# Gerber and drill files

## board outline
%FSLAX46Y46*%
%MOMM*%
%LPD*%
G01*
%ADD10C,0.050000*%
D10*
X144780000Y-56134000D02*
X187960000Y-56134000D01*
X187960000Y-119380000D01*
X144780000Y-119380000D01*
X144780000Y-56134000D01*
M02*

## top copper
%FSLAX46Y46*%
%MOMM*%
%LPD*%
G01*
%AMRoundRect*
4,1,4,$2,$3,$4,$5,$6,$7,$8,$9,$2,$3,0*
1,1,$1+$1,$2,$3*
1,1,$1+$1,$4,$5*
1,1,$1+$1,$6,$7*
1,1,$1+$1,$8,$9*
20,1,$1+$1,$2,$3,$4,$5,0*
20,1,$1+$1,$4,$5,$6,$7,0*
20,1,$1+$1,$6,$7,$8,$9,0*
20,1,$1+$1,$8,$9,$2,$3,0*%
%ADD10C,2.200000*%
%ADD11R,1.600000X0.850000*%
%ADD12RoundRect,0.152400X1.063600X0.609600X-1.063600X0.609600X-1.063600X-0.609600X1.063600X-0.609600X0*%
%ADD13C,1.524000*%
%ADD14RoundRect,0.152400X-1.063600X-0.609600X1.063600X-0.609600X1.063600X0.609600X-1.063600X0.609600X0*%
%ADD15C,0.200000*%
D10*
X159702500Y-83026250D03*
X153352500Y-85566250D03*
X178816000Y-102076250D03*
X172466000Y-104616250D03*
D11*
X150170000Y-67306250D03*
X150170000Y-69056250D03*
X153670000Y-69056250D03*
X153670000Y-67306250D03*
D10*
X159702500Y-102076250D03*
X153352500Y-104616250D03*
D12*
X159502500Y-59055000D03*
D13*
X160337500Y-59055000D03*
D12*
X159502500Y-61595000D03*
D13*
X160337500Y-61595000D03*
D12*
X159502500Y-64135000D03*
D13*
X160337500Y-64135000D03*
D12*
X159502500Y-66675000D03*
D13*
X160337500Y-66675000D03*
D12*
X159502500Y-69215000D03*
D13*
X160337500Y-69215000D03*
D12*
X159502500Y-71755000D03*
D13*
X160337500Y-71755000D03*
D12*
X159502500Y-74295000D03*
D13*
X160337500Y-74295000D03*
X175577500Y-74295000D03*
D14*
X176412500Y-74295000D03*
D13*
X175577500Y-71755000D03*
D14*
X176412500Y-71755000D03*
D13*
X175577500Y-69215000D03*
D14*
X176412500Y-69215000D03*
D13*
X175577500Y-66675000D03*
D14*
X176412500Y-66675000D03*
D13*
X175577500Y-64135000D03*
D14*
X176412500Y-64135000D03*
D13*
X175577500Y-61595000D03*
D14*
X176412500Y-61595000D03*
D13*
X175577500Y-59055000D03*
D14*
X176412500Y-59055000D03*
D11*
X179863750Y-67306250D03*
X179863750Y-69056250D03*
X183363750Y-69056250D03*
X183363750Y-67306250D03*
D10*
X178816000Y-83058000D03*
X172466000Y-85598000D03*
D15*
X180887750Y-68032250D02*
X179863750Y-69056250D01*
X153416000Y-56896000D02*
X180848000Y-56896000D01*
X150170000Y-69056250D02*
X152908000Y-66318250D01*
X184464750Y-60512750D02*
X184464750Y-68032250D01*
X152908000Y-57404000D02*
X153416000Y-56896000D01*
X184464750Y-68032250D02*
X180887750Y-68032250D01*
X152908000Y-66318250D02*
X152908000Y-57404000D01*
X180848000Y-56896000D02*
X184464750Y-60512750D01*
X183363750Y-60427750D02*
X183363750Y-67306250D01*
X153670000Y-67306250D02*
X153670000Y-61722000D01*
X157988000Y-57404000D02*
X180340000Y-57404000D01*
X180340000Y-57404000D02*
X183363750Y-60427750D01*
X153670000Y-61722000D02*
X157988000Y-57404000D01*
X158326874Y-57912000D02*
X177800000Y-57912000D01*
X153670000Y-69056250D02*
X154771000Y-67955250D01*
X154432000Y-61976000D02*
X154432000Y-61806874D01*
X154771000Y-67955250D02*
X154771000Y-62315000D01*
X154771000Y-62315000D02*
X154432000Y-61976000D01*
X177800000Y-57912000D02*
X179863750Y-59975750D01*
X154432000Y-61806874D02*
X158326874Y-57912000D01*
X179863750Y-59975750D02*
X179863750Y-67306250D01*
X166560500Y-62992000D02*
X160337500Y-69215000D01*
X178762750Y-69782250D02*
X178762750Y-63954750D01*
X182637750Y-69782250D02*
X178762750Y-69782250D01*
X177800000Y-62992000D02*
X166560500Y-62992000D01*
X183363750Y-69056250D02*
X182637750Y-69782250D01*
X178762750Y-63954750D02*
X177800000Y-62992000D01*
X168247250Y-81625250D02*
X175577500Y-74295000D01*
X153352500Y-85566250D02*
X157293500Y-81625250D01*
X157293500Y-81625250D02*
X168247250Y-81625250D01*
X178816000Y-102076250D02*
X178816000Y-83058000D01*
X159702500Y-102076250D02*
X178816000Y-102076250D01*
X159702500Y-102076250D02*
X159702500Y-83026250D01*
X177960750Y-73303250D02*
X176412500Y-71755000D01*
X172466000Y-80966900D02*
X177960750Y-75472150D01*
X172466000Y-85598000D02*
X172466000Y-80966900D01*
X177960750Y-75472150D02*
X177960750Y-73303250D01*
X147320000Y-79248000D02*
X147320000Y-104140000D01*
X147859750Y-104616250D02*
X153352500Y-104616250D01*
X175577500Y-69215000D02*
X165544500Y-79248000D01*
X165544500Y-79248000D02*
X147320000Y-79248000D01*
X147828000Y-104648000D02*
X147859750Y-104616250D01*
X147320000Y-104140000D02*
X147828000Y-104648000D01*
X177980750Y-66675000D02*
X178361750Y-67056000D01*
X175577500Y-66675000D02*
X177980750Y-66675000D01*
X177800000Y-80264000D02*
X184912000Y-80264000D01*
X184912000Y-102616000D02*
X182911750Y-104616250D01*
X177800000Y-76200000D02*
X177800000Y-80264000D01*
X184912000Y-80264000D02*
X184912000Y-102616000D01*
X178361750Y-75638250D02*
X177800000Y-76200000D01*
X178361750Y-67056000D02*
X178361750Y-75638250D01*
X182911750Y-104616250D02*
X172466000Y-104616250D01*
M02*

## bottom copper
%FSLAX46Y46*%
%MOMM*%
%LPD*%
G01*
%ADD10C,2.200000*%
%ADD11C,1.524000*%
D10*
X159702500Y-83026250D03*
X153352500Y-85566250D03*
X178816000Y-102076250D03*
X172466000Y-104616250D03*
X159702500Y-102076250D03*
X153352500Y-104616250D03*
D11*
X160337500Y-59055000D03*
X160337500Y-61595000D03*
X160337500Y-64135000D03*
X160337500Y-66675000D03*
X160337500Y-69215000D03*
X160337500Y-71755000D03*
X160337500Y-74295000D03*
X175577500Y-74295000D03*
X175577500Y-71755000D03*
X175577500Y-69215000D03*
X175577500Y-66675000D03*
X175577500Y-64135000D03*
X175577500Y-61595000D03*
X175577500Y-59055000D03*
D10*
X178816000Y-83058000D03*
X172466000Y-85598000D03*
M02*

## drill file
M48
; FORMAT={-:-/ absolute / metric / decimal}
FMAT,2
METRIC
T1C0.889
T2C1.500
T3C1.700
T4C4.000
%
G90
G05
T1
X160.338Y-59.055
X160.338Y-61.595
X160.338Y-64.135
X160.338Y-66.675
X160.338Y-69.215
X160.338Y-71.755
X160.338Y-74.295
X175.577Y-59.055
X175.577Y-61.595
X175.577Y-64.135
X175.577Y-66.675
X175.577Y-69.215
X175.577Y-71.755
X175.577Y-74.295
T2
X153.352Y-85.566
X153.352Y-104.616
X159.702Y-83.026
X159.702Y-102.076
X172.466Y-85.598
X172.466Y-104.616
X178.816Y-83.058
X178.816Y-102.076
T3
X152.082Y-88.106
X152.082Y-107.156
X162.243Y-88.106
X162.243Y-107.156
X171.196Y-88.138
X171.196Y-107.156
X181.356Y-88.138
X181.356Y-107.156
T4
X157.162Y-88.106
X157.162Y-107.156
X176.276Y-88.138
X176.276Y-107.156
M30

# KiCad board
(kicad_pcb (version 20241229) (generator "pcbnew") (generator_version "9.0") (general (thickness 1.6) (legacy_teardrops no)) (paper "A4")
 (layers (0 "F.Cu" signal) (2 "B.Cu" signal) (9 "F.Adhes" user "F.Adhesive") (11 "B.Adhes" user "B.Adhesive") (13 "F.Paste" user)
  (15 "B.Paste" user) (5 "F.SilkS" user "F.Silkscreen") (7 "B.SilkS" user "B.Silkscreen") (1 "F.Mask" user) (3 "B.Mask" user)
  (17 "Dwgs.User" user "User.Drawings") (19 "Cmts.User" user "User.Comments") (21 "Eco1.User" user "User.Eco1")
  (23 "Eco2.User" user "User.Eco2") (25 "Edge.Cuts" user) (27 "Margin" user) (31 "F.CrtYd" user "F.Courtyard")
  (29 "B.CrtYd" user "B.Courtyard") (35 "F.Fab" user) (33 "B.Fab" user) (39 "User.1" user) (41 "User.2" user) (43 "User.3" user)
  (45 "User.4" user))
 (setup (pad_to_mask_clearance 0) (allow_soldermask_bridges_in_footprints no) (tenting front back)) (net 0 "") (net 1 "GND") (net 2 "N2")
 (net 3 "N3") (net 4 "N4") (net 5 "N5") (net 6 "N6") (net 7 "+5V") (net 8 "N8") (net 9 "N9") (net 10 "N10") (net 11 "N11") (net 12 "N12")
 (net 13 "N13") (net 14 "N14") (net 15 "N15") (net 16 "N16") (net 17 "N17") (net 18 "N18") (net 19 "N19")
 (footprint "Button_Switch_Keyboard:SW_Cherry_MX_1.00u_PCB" (layer "F.Cu") (at 159.7025 83.02625)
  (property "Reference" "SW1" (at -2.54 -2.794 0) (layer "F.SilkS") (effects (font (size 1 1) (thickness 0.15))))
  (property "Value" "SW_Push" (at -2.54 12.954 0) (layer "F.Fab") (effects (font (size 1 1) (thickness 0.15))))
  (pad "" np_thru_hole circle (at -7.62 5.08) (size 1.7 1.7) (drill 1.7) (layers "*.Cu" "*.Mask"))
  (pad "" np_thru_hole circle (at -2.54 5.08) (size 4 4) (drill 4) (layers "*.Cu" "*.Mask"))
  (pad "" np_thru_hole circle (at 2.54 5.08) (size 1.7 1.7) (drill 1.7) (layers "*.Cu" "*.Mask"))
  (pad "1" thru_hole circle (at 0 0) (size 2.2 2.2) (drill 1.5) (layers "*.Cu" "*.Mask") (remove_unused_layers no) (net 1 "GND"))
  (pad "2" thru_hole circle (at -6.35 2.54) (size 2.2 2.2) (drill 1.5) (layers "*.Cu" "*.Mask") (remove_unused_layers no) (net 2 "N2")))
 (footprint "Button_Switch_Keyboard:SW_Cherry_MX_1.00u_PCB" (layer "F.Cu") (at 178.816 102.07625)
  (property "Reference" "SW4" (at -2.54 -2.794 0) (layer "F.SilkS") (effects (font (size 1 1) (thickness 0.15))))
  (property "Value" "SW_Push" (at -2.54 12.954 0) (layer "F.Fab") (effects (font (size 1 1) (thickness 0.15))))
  (pad "" np_thru_hole circle (at -7.62 5.08) (size 1.7 1.7) (drill 1.7) (layers "*.Cu" "*.Mask"))
  (pad "" np_thru_hole circle (at -2.54 5.08) (size 4 4) (drill 4) (layers "*.Cu" "*.Mask"))
  (pad "" np_thru_hole circle (at 2.54 5.08) (size 1.7 1.7) (drill 1.7) (layers "*.Cu" "*.Mask"))
  (pad "1" thru_hole circle (at 0 0) (size 2.2 2.2) (drill 1.5) (layers "*.Cu" "*.Mask") (remove_unused_layers no) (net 1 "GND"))
  (pad "2" thru_hole circle (at -6.35 2.54) (size 2.2 2.2) (drill 1.5) (layers "*.Cu" "*.Mask") (remove_unused_layers no) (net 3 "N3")))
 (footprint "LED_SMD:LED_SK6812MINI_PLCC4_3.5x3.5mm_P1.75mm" (layer "F.Cu") (at 151.92 68.18125)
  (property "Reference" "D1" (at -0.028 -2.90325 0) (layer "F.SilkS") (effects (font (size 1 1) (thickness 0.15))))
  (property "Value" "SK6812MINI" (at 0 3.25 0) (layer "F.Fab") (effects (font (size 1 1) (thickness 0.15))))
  (pad "1" smd rect (at -1.75 -0.875) (size 1.6 0.85) (layers "F.Cu" "F.Mask" "F.Paste") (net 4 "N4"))
  (pad "2" smd rect (at -1.75 0.875) (size 1.6 0.85) (layers "F.Cu" "F.Mask" "F.Paste") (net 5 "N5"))
  (pad "3" smd rect (at 1.75 0.875) (size 1.6 0.85) (layers "F.Cu" "F.Mask" "F.Paste") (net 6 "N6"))
  (pad "4" smd rect (at 1.75 -0.875) (size 1.6 0.85) (layers "F.Cu" "F.Mask" "F.Paste") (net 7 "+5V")))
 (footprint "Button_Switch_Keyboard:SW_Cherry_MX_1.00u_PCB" (layer "F.Cu") (at 159.7025 102.07625)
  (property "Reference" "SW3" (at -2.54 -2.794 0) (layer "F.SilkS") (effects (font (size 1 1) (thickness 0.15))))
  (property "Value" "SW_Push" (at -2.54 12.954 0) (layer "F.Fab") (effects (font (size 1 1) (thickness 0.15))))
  (pad "" np_thru_hole circle (at -7.62 5.08) (size 1.7 1.7) (drill 1.7) (layers "*.Cu" "*.Mask"))
  (pad "" np_thru_hole circle (at -2.54 5.08) (size 4 4) (drill 4) (layers "*.Cu" "*.Mask"))
  (pad "" np_thru_hole circle (at 2.54 5.08) (size 1.7 1.7) (drill 1.7) (layers "*.Cu" "*.Mask"))
  (pad "1" thru_hole circle (at 0 0) (size 2.2 2.2) (drill 1.5) (layers "*.Cu" "*.Mask") (remove_unused_layers no) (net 1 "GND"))
  (pad "2" thru_hole circle (at -6.35 2.54) (size 2.2 2.2) (drill 1.5) (layers "*.Cu" "*.Mask") (remove_unused_layers no) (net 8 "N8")))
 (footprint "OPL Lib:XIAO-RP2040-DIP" (layer "F.Cu") (at 167.9575 66.675)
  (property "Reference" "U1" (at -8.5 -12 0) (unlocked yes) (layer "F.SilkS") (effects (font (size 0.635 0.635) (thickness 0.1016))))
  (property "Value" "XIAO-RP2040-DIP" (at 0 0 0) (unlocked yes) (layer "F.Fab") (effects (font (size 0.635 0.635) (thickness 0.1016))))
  (pad "1" smd roundrect (at -8.455 -7.62 180) (size 2.432 1.524) (layers "F.Cu" "F.Mask") (roundrect_rratio 0.1) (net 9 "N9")
   (thermal_bridge_angle 45))
  (pad "1" thru_hole circle (at -7.62 -7.62 180) (size 1.524 1.524) (drill 0.889) (layers "*.Cu" "*.Mask") (remove_unused_layers no)
   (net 9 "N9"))
  (pad "2" smd roundrect (at -8.455 -5.08 180) (size 2.432 1.524) (layers "F.Cu" "F.Mask") (roundrect_rratio 0.1) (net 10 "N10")
   (thermal_bridge_angle 45))
  (pad "2" thru_hole circle (at -7.62 -5.08 180) (size 1.524 1.524) (drill 0.889) (layers "*.Cu" "*.Mask") (remove_unused_layers no)
   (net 10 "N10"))
  (pad "3" smd roundrect (at -8.455 -2.54 180) (size 2.432 1.524) (layers "F.Cu" "F.Mask") (roundrect_rratio 0.1) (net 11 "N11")
   (thermal_bridge_angle 45))
  (pad "3" thru_hole circle (at -7.62 -2.54 180) (size 1.524 1.524) (drill 0.889) (layers "*.Cu" "*.Mask") (remove_unused_layers no)
   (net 11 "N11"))
  (pad "4" smd roundrect (at -8.455 0 180) (size 2.432 1.524) (layers "F.Cu" "F.Mask") (roundrect_rratio 0.1) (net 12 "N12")
   (thermal_bridge_angle 45))
  (pad "4" thru_hole circle (at -7.62 0 180) (size 1.524 1.524) (drill 0.889) (layers "*.Cu" "*.Mask") (remove_unused_layers no)
   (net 12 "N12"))
  (pad "5" smd roundrect (at -8.455 2.54 180) (size 2.432 1.524) (layers "F.Cu" "F.Mask") (roundrect_rratio 0.1) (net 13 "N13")
   (thermal_bridge_angle 45))
  (pad "5" thru_hole circle (at -7.62 2.54 180) (size 1.524 1.524) (drill 0.889) (layers "*.Cu" "*.Mask") (remove_unused_layers no)
   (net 13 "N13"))
  (pad "6" smd roundrect (at -8.455 5.08 180) (size 2.432 1.524) (layers "F.Cu" "F.Mask") (roundrect_rratio 0.1) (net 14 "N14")
   (thermal_bridge_angle 45))
  (pad "6" thru_hole circle (at -7.62 5.08 180) (size 1.524 1.524) (drill 0.889) (layers "*.Cu" "*.Mask") (remove_unused_layers no)
   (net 14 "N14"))
  (pad "7" smd roundrect (at -8.455 7.62 180) (size 2.432 1.524) (layers "F.Cu" "F.Mask") (roundrect_rratio 0.1) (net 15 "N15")
   (thermal_bridge_angle 45))
  (pad "7" thru_hole circle (at -7.62 7.62 180) (size 1.524 1.524) (drill 0.889) (layers "*.Cu" "*.Mask") (remove_unused_layers no)
   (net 15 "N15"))
  (pad "8" thru_hole circle (at 7.62 7.62) (size 1.524 1.524) (drill 0.889) (layers "*.Cu" "*.Mask") (remove_unused_layers no) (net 2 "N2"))
  (pad "8" smd roundrect (at 8.455 7.62) (size 2.432 1.524) (layers "F.Cu" "F.Mask") (roundrect_rratio 0.1) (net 2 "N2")
   (thermal_bridge_angle 45))
  (pad "9" thru_hole circle (at 7.62 5.08) (size 1.524 1.524) (drill 0.889) (layers "*.Cu" "*.Mask") (remove_unused_layers no)
   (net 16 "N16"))
  (pad "9" smd roundrect (at 8.455 5.08) (size 2.432 1.524) (layers "F.Cu" "F.Mask") (roundrect_rratio 0.1) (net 16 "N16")
   (thermal_bridge_angle 45))
  (pad "10" thru_hole circle (at 7.62 2.54) (size 1.524 1.524) (drill 0.889) (layers "*.Cu" "*.Mask") (remove_unused_layers no) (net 8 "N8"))
  (pad "10" smd roundrect (at 8.455 2.54) (size 2.432 1.524) (layers "F.Cu" "F.Mask") (roundrect_rratio 0.1) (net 8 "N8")
   (thermal_bridge_angle 45))
  (pad "11" thru_hole circle (at 7.62 0) (size 1.524 1.524) (drill 0.889) (layers "*.Cu" "*.Mask") (remove_unused_layers no) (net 3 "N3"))
  (pad "11" smd roundrect (at 8.455 0) (size 2.432 1.524) (layers "F.Cu" "F.Mask") (roundrect_rratio 0.1) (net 3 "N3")
   (thermal_bridge_angle 45))
  (pad "12" thru_hole circle (at 7.62 -2.54) (size 1.524 1.524) (drill 0.889) (layers "*.Cu" "*.Mask") (remove_unused_layers no)
   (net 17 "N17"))
  (pad "12" smd roundrect (at 8.455 -2.54) (size 2.432 1.524) (layers "F.Cu" "F.Mask") (roundrect_rratio 0.1) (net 17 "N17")
   (thermal_bridge_angle 45))
  (pad "13" thru_hole circle (at 7.62 -5.08) (size 1.524 1.524) (drill 0.889) (layers "*.Cu" "*.Mask") (remove_unused_layers no)
   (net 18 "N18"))
  (pad "13" smd roundrect (at 8.455 -5.08) (size 2.432 1.524) (layers "F.Cu" "F.Mask") (roundrect_rratio 0.1) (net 18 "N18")
   (thermal_bridge_angle 45))
  (pad "14" thru_hole circle (at 7.62 -7.62) (size 1.524 1.524) (drill 0.889) (layers "*.Cu" "*.Mask") (remove_unused_layers no)
   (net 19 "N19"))
  (pad "14" smd roundrect (at 8.455 -7.62) (size 2.432 1.524) (layers "F.Cu" "F.Mask") (roundrect_rratio 0.1) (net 19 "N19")
   (thermal_bridge_angle 45)))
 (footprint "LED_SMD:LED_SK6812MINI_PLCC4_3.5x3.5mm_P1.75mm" (layer "F.Cu") (at 181.61375 68.18125)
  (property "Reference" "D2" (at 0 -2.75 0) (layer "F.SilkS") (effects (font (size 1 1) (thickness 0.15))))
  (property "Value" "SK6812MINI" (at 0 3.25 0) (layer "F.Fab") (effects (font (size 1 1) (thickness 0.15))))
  (pad "1" smd rect (at -1.75 -0.875) (size 1.6 0.85) (layers "F.Cu" "F.Mask" "F.Paste") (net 6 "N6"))
  (pad "2" smd rect (at -1.75 0.875) (size 1.6 0.85) (layers "F.Cu" "F.Mask" "F.Paste") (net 5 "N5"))
  (pad "3" smd rect (at 1.75 0.875) (size 1.6 0.85) (layers "F.Cu" "F.Mask" "F.Paste") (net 13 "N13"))
  (pad "4" smd rect (at 1.75 -0.875) (size 1.6 0.85) (layers "F.Cu" "F.Mask" "F.Paste") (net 7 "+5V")))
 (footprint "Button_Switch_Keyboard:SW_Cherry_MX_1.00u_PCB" (layer "F.Cu") (at 178.816 83.058)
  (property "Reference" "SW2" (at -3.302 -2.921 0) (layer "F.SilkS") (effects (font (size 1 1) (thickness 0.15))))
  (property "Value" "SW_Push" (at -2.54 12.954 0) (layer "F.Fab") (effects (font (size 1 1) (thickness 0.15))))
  (pad "" np_thru_hole circle (at -7.62 5.08) (size 1.7 1.7) (drill 1.7) (layers "*.Cu" "*.Mask"))
  (pad "" np_thru_hole circle (at -2.54 5.08) (size 4 4) (drill 4) (layers "*.Cu" "*.Mask"))
  (pad "" np_thru_hole circle (at 2.54 5.08) (size 1.7 1.7) (drill 1.7) (layers "*.Cu" "*.Mask"))
  (pad "1" thru_hole circle (at 0 0) (size 2.2 2.2) (drill 1.5) (layers "*.Cu" "*.Mask") (remove_unused_layers no) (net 1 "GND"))
  (pad "2" thru_hole circle (at -6.35 2.54) (size 2.2 2.2) (drill 1.5) (layers "*.Cu" "*.Mask") (remove_unused_layers no) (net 16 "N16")))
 (gr_rect (start 144.78 56.134) (end 187.96 119.38) (stroke (width 0.05) (type default)) (fill no) (layer "Edge.Cuts"))
 (segment (start 180.88775 68.03225) (end 179.86375 69.05625) (width 0.2) (layer "F.Cu") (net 5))
 (segment (start 153.416 56.896) (end 180.848 56.896) (width 0.2) (layer "F.Cu") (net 5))
 (segment (start 150.17 69.05625) (end 152.908 66.31825) (width 0.2) (layer "F.Cu") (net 5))
 (segment (start 184.46475 60.51275) (end 184.46475 68.03225) (width 0.2) (layer "F.Cu") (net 5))
 (segment (start 152.908 57.404) (end 153.416 56.896) (width 0.2) (layer "F.Cu") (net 5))
 (segment (start 184.46475 68.03225) (end 180.88775 68.03225) (width 0.2) (layer "F.Cu") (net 5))
 (segment (start 152.908 66.31825) (end 152.908 57.404) (width 0.2) (layer "F.Cu") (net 5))
 (segment (start 180.848 56.896) (end 184.46475 60.51275) (width 0.2) (layer "F.Cu") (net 5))
 (segment (start 183.36375 60.42775) (end 183.36375 67.30625) (width 0.2) (layer "F.Cu") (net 7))
 (segment (start 153.67 67.30625) (end 153.67 61.722) (width 0.2) (layer "F.Cu") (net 7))
 (segment (start 157.988 57.404) (end 180.34 57.404) (width 0.2) (layer "F.Cu") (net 7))
 (segment (start 180.34 57.404) (end 183.36375 60.42775) (width 0.2) (layer "F.Cu") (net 7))
 (segment (start 153.67 61.722) (end 157.988 57.404) (width 0.2) (layer "F.Cu") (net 7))
 (segment (start 158.326874 57.912) (end 177.8 57.912) (width 0.2) (layer "F.Cu") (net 6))
 (segment (start 153.67 69.05625) (end 154.771 67.95525) (width 0.2) (layer "F.Cu") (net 6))
 (segment (start 154.432 61.976) (end 154.432 61.806874) (width 0.2) (layer "F.Cu") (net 6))
 (segment (start 154.771 67.95525) (end 154.771 62.315) (width 0.2) (layer "F.Cu") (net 6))
 (segment (start 154.771 62.315) (end 154.432 61.976) (width 0.2) (layer "F.Cu") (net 6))
 (segment (start 177.8 57.912) (end 179.86375 59.97575) (width 0.2) (layer "F.Cu") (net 6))
 (segment (start 154.432 61.806874) (end 158.326874 57.912) (width 0.2) (layer "F.Cu") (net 6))
 (segment (start 179.86375 59.97575) (end 179.86375 67.30625) (width 0.2) (layer "F.Cu") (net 6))
 (segment (start 166.5605 62.992) (end 160.3375 69.215) (width 0.2) (layer "F.Cu") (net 13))
 (segment (start 178.76275 69.78225) (end 178.76275 63.95475) (width 0.2) (layer "F.Cu") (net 13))
 (segment (start 182.63775 69.78225) (end 178.76275 69.78225) (width 0.2) (layer "F.Cu") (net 13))
 (segment (start 177.8 62.992) (end 166.5605 62.992) (width 0.2) (layer "F.Cu") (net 13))
 (segment (start 183.36375 69.05625) (end 182.63775 69.78225) (width 0.2) (layer "F.Cu") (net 13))
 (segment (start 178.76275 63.95475) (end 177.8 62.992) (width 0.2) (layer "F.Cu") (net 13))
 (segment (start 168.24725 81.62525) (end 175.5775 74.295) (width 0.2) (layer "F.Cu") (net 2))
 (segment (start 153.3525 85.56625) (end 157.2935 81.62525) (width 0.2) (layer "F.Cu") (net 2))
 (segment (start 157.2935 81.62525) (end 168.24725 81.62525) (width 0.2) (layer "F.Cu") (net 2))
 (segment (start 178.816 102.07625) (end 178.816 83.058) (width 0.2) (layer "F.Cu") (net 1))
 (segment (start 159.7025 102.07625) (end 178.816 102.07625) (width 0.2) (layer "F.Cu") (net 1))
 (segment (start 159.7025 102.07625) (end 159.7025 83.02625) (width 0.2) (layer "F.Cu") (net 1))
 (segment (start 177.96075 73.30325) (end 176.4125 71.755) (width 0.2) (layer "F.Cu") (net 16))
 (segment (start 172.466 80.9669) (end 177.96075 75.47215) (width 0.2) (layer "F.Cu") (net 16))
 (segment (start 172.466 85.598) (end 172.466 80.9669) (width 0.2) (layer "F.Cu") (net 16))
 (segment (start 177.96075 75.47215) (end 177.96075 73.30325) (width 0.2) (layer "F.Cu") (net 16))
 (segment (start 147.32 79.248) (end 147.32 104.14) (width 0.2) (layer "F.Cu") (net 8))
 (segment (start 147.85975 104.61625) (end 153.3525 104.61625) (width 0.2) (layer "F.Cu") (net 8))
 (segment (start 175.5775 69.215) (end 165.5445 79.248) (width 0.2) (layer "F.Cu") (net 8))
 (segment (start 165.5445 79.248) (end 147.32 79.248) (width 0.2) (layer "F.Cu") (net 8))
 (segment (start 147.828 104.648) (end 147.85975 104.61625) (width 0.2) (layer "F.Cu") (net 8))
 (segment (start 147.32 104.14) (end 147.828 104.648) (width 0.2) (layer "F.Cu") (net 8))
 (segment (start 177.98075 66.675) (end 178.36175 67.056) (width 0.2) (layer "F.Cu") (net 3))
 (segment (start 175.5775 66.675) (end 177.98075 66.675) (width 0.2) (layer "F.Cu") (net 3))
 (segment (start 177.8 80.264) (end 184.912 80.264) (width 0.2) (layer "F.Cu") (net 3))
 (segment (start 184.912 102.616) (end 182.91175 104.61625) (width 0.2) (layer "F.Cu") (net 3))
 (segment (start 177.8 76.2) (end 177.8 80.264) (width 0.2) (layer "F.Cu") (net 3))
 (segment (start 184.912 80.264) (end 184.912 102.616) (width 0.2) (layer "F.Cu") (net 3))
 (segment (start 178.36175 75.63825) (end 177.8 76.2) (width 0.2) (layer "F.Cu") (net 3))
 (segment (start 178.36175 67.056) (end 178.36175 75.63825) (width 0.2) (layer "F.Cu") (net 3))
 (segment (start 182.91175 104.61625) (end 172.466 104.61625) (width 0.2) (layer "F.Cu") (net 3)))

